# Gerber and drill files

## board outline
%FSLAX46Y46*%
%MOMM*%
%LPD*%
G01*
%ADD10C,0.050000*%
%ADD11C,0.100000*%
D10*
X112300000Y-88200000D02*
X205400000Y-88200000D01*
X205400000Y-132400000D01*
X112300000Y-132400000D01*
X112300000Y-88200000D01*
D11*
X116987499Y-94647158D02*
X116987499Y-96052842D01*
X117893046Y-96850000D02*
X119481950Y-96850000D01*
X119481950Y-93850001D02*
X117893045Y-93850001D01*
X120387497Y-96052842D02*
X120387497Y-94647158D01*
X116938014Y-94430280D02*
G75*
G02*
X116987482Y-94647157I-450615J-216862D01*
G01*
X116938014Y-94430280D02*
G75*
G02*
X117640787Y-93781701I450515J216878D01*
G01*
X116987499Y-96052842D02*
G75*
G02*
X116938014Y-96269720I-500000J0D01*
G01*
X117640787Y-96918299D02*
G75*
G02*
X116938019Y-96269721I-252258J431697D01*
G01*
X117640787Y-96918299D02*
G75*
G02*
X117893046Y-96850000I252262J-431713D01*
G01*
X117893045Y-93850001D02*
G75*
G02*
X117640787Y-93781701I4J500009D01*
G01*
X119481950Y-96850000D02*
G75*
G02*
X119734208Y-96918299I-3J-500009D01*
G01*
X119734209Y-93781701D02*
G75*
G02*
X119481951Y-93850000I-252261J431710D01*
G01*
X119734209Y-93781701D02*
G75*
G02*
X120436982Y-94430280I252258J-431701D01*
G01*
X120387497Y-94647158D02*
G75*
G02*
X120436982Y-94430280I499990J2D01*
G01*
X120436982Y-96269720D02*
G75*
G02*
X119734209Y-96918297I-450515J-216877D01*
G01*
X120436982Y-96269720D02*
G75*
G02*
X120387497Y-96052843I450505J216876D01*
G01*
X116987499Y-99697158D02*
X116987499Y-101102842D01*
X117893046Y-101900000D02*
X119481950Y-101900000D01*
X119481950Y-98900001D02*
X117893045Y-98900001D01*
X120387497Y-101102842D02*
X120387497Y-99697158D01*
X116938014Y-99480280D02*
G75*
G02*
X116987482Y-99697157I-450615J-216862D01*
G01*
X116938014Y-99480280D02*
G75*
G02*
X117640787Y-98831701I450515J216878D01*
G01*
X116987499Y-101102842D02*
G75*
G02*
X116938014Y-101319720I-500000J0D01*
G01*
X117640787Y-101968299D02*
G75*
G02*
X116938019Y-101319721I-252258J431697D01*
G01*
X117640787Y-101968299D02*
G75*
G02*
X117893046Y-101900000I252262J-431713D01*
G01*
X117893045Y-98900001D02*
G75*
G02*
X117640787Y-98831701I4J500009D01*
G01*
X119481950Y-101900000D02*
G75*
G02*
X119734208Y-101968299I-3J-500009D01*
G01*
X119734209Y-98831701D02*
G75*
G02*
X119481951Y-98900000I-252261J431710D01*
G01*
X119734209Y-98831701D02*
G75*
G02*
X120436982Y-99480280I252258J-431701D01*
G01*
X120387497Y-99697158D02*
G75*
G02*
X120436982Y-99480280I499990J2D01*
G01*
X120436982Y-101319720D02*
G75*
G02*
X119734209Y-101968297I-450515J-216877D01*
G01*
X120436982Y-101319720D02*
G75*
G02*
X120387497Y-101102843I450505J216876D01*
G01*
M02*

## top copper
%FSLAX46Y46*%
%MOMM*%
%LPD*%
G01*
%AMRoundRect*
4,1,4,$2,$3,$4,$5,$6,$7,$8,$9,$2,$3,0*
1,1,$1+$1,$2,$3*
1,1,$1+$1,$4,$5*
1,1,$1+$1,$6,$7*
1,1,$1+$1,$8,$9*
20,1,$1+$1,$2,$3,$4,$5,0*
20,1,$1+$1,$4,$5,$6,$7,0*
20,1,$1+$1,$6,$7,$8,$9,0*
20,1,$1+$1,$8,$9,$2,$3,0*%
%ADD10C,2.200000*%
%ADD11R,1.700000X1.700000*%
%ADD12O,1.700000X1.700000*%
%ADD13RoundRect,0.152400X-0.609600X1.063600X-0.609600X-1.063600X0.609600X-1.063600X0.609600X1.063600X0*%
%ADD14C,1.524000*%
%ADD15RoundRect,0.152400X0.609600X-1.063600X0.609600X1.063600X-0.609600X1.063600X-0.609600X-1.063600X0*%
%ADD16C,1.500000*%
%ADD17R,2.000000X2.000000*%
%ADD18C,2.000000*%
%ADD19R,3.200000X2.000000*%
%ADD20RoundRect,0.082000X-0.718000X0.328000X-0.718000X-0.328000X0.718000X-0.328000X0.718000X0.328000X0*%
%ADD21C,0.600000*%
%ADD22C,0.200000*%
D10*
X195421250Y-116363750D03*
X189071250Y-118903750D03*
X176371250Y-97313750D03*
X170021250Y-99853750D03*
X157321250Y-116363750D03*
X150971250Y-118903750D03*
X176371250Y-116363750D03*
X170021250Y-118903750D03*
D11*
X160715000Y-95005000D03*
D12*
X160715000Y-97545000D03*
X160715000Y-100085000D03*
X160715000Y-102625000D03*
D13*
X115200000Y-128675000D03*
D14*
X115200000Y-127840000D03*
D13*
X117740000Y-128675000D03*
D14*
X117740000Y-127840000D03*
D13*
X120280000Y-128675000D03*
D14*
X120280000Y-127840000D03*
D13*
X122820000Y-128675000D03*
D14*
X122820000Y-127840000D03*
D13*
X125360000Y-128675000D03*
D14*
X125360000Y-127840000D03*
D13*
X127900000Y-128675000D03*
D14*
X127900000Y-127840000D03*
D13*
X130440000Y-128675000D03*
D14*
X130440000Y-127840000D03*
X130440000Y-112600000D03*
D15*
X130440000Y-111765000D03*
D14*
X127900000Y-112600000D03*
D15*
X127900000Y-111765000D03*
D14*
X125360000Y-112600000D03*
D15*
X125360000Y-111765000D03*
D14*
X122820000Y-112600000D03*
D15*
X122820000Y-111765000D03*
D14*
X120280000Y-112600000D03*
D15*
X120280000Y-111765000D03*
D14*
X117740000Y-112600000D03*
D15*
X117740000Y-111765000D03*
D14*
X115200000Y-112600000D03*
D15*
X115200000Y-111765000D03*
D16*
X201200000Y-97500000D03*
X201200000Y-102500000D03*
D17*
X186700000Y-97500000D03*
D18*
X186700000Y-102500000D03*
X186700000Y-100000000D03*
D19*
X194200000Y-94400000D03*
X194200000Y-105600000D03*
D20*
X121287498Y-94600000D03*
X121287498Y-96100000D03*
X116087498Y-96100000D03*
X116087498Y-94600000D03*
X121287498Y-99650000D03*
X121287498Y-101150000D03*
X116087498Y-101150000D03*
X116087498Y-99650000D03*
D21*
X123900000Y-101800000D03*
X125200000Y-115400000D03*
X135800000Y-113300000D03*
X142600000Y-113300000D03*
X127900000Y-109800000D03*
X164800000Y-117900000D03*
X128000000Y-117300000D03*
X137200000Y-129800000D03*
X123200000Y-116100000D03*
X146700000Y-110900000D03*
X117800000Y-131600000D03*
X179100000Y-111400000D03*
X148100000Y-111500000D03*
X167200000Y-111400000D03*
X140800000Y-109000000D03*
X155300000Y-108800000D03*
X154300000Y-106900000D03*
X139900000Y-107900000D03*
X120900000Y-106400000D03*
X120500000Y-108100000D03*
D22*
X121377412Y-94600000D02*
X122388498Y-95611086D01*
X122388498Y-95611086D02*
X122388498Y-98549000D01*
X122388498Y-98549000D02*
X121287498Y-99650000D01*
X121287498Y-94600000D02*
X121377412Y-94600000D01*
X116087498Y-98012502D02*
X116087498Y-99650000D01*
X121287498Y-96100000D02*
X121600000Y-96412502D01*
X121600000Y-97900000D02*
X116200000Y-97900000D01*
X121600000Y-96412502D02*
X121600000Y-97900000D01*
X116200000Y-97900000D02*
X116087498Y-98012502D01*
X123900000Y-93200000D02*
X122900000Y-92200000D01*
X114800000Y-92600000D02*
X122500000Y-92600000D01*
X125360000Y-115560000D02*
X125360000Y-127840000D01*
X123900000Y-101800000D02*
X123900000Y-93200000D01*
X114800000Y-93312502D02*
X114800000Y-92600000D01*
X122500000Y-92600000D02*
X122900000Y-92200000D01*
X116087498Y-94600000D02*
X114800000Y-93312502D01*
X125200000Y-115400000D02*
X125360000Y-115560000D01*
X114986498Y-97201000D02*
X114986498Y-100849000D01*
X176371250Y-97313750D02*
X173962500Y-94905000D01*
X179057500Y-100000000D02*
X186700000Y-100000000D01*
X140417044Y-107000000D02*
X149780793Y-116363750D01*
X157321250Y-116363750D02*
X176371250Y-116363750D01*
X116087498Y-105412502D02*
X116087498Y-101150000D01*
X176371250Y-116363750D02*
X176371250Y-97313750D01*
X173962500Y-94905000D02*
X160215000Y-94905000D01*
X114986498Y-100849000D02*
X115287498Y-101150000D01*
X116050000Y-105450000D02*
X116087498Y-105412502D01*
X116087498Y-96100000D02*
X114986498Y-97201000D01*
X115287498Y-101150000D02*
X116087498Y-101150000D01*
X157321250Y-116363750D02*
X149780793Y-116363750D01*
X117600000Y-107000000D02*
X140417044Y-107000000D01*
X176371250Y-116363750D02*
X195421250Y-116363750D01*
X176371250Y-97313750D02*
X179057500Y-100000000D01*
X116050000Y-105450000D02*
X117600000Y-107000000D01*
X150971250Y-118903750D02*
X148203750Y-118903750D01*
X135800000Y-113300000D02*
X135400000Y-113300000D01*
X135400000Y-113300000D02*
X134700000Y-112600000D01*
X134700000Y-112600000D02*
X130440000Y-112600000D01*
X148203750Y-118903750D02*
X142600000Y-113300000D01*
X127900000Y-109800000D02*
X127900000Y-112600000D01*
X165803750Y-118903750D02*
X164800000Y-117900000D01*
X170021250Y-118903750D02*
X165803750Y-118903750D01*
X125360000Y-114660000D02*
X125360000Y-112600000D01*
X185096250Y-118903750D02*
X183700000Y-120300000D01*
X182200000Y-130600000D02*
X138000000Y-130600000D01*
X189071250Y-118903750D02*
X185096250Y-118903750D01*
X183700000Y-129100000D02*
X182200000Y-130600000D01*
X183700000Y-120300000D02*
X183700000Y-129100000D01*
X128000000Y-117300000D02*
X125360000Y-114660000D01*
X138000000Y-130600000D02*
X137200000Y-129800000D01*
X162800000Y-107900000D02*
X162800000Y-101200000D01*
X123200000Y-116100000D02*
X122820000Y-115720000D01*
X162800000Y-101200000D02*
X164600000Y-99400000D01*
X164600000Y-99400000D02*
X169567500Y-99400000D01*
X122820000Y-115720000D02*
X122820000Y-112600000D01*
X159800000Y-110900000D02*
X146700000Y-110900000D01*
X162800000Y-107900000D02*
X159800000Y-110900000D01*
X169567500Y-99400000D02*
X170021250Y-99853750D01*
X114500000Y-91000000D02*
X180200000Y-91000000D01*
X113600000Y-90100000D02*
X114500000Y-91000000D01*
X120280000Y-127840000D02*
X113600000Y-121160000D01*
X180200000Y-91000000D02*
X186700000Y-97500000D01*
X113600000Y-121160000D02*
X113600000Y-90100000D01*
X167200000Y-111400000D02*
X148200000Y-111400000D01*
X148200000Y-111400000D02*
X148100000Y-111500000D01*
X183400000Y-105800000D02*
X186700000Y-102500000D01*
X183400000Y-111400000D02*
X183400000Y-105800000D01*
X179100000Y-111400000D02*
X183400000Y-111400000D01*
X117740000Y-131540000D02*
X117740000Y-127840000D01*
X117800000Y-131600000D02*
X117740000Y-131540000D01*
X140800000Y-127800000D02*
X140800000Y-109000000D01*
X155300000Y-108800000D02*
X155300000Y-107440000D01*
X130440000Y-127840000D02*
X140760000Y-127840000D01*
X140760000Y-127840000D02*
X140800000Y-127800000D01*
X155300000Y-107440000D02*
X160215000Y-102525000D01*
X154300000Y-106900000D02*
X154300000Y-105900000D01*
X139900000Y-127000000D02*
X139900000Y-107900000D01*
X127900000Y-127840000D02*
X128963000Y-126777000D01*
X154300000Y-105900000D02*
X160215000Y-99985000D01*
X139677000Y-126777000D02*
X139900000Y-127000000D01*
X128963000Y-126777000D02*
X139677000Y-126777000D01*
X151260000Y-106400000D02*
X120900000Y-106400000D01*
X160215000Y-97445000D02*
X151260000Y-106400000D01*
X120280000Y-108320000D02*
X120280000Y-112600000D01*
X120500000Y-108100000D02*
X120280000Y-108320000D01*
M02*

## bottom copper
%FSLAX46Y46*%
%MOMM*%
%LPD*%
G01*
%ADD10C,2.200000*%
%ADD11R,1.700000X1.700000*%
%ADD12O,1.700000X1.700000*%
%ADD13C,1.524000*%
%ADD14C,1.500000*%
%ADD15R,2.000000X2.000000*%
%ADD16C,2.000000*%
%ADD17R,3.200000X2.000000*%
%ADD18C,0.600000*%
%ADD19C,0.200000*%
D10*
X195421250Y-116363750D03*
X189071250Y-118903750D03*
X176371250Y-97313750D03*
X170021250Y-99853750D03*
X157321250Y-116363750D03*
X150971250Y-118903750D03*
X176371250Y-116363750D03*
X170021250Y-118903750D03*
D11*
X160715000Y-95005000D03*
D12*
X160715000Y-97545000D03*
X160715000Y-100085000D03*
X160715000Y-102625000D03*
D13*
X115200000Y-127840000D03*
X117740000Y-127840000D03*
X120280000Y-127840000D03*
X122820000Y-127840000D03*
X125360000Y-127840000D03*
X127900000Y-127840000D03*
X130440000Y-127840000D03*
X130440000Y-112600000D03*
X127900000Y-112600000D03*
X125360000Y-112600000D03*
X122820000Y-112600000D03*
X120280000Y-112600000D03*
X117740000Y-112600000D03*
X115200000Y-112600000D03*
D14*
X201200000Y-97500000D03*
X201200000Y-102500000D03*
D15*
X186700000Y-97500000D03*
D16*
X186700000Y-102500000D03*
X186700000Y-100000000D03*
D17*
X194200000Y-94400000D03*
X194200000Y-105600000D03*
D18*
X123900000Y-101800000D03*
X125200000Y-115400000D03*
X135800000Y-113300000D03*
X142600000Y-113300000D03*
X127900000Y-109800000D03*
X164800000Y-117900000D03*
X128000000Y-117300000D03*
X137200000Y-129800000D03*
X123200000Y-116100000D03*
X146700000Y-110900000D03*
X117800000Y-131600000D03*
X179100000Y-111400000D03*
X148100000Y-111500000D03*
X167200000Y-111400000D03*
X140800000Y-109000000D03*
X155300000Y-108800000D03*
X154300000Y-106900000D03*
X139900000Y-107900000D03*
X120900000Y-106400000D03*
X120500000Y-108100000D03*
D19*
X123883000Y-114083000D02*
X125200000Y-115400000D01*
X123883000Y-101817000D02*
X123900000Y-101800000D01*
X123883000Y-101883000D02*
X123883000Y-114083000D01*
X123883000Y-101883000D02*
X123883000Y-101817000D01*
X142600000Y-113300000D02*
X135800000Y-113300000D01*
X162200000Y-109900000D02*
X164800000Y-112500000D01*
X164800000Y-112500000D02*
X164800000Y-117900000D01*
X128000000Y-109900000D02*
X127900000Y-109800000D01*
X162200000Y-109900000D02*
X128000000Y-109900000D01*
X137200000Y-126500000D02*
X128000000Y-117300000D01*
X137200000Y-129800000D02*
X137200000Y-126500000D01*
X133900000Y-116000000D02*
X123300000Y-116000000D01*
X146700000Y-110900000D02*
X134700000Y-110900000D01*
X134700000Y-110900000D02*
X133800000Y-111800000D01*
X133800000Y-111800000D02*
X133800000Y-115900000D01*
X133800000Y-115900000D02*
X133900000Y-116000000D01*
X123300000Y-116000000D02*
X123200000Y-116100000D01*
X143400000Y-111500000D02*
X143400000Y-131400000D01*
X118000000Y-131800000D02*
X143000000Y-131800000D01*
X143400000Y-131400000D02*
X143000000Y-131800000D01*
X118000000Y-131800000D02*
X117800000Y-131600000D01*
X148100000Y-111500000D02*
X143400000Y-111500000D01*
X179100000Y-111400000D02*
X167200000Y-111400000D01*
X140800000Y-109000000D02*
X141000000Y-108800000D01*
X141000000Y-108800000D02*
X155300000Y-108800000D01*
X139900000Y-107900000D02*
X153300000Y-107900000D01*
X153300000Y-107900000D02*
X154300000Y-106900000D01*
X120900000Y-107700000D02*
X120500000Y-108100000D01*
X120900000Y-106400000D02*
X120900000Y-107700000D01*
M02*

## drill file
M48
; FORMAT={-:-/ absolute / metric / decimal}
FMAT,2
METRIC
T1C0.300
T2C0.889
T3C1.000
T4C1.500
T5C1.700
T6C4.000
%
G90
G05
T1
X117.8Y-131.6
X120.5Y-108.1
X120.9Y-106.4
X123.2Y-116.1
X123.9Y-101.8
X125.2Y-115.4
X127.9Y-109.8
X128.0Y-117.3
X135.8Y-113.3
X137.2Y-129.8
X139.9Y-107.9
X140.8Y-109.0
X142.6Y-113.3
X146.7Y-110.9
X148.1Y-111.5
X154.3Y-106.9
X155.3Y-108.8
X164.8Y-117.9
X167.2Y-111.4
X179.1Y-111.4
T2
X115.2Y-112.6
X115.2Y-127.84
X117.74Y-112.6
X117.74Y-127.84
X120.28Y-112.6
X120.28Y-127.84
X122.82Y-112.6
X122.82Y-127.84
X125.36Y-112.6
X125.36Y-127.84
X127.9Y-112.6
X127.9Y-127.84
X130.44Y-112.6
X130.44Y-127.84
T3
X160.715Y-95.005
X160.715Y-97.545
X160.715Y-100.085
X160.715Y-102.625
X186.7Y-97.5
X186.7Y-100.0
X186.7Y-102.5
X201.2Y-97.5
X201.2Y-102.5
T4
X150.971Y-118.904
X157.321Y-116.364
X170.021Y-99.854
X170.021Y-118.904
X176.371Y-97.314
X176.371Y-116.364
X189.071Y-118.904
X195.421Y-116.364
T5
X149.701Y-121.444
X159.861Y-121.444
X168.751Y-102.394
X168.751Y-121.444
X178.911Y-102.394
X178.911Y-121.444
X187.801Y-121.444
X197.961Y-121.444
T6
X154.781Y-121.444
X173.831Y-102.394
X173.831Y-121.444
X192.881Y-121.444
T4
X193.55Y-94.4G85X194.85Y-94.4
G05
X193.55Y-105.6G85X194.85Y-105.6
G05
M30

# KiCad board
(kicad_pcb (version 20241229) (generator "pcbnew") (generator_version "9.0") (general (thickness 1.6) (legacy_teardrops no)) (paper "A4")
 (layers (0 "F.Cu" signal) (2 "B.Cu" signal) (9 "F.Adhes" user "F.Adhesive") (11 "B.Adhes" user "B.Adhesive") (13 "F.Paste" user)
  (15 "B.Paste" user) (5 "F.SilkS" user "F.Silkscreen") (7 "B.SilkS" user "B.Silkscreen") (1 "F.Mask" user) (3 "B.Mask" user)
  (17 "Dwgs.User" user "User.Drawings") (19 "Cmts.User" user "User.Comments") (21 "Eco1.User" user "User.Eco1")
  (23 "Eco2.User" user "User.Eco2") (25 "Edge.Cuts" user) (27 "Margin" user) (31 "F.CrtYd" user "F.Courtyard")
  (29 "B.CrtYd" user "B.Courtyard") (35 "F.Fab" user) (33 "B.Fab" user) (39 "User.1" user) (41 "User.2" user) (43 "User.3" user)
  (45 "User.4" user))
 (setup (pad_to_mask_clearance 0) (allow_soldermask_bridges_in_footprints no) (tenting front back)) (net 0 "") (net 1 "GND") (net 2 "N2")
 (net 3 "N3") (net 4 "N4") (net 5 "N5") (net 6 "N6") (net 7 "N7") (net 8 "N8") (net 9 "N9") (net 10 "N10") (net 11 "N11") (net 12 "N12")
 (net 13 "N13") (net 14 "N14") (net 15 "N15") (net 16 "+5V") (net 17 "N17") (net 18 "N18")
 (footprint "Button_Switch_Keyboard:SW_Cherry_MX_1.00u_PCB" (layer "F.Cu") (at 195.42125 116.36375)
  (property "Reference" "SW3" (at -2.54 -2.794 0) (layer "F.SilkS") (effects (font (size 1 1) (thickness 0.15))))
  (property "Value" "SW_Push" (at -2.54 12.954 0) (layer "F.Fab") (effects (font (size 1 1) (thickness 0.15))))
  (pad "" np_thru_hole circle (at -7.62 5.08) (size 1.7 1.7) (drill 1.7) (layers "*.Cu" "*.Mask"))
  (pad "" np_thru_hole circle (at -2.54 5.08) (size 4 4) (drill 4) (layers "*.Cu" "*.Mask"))
  (pad "" np_thru_hole circle (at 2.54 5.08) (size 1.7 1.7) (drill 1.7) (layers "*.Cu" "*.Mask"))
  (pad "1" thru_hole circle (at 0 0) (size 2.2 2.2) (drill 1.5) (layers "*.Cu" "*.Mask") (remove_unused_layers no) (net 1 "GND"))
  (pad "2" thru_hole circle (at -6.35 2.54) (size 2.2 2.2) (drill 1.5) (layers "*.Cu" "*.Mask") (remove_unused_layers no) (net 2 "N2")))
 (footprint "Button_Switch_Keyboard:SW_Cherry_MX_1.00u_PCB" (layer "F.Cu") (at 176.37125 97.31375)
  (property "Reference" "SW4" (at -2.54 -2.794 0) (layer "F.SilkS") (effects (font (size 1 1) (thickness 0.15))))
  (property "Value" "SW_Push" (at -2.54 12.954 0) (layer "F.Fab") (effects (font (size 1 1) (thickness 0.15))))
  (pad "" np_thru_hole circle (at -7.62 5.08) (size 1.7 1.7) (drill 1.7) (layers "*.Cu" "*.Mask"))
  (pad "" np_thru_hole circle (at -2.54 5.08) (size 4 4) (drill 4) (layers "*.Cu" "*.Mask"))
  (pad "" np_thru_hole circle (at 2.54 5.08) (size 1.7 1.7) (drill 1.7) (layers "*.Cu" "*.Mask"))
  (pad "1" thru_hole circle (at 0 0) (size 2.2 2.2) (drill 1.5) (layers "*.Cu" "*.Mask") (remove_unused_layers no) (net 1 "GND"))
  (pad "2" thru_hole circle (at -6.35 2.54) (size 2.2 2.2) (drill 1.5) (layers "*.Cu" "*.Mask") (remove_unused_layers no) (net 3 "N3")))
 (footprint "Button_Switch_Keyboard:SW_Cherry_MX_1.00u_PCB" (layer "F.Cu") (at 157.32125 116.36375)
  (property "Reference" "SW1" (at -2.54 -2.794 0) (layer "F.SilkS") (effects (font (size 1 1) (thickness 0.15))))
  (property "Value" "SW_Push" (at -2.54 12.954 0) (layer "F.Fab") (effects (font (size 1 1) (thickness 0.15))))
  (pad "" np_thru_hole circle (at -7.62 5.08) (size 1.7 1.7) (drill 1.7) (layers "*.Cu" "*.Mask"))
  (pad "" np_thru_hole circle (at -2.54 5.08) (size 4 4) (drill 4) (layers "*.Cu" "*.Mask"))
  (pad "" np_thru_hole circle (at 2.54 5.08) (size 1.7 1.7) (drill 1.7) (layers "*.Cu" "*.Mask"))
  (pad "1" thru_hole circle (at 0 0) (size 2.2 2.2) (drill 1.5) (layers "*.Cu" "*.Mask") (remove_unused_layers no) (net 1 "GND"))
  (pad "2" thru_hole circle (at -6.35 2.54) (size 2.2 2.2) (drill 1.5) (layers "*.Cu" "*.Mask") (remove_unused_layers no) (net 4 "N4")))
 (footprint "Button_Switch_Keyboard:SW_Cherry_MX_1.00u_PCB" (layer "F.Cu") (at 176.37125 116.36375)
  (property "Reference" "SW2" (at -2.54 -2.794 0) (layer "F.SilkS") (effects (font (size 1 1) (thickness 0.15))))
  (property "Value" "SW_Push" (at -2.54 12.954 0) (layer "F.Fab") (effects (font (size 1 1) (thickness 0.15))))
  (pad "" np_thru_hole circle (at -7.62 5.08) (size 1.7 1.7) (drill 1.7) (layers "*.Cu" "*.Mask"))
  (pad "" np_thru_hole circle (at -2.54 5.08) (size 4 4) (drill 4) (layers "*.Cu" "*.Mask"))
  (pad "" np_thru_hole circle (at 2.54 5.08) (size 1.7 1.7) (drill 1.7) (layers "*.Cu" "*.Mask"))
  (pad "1" thru_hole circle (at 0 0) (size 2.2 2.2) (drill 1.5) (layers "*.Cu" "*.Mask") (remove_unused_layers no) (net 1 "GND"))
  (pad "2" thru_hole circle (at -6.35 2.54) (size 2.2 2.2) (drill 1.5) (layers "*.Cu" "*.Mask") (remove_unused_layers no) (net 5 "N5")))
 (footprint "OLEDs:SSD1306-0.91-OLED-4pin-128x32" (layer "F.Cu") (at 124.215 92.815)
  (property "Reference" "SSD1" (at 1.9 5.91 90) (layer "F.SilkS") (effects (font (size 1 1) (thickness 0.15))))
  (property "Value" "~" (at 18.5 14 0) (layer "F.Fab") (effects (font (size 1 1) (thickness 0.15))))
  (pad "1" thru_hole rect (at 36.5 2.19) (size 1.7 1.7) (drill 1) (layers "*.Cu" "*.Mask") (remove_unused_layers no) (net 1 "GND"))
  (pad "2" thru_hole oval (at 36.5 4.73) (size 1.7 1.7) (drill 1) (layers "*.Cu" "*.Mask") (remove_unused_layers no) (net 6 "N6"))
  (pad "3" thru_hole oval (at 36.5 7.27) (size 1.7 1.7) (drill 1) (layers "*.Cu" "*.Mask") (remove_unused_layers no) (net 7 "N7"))
  (pad "4" thru_hole oval (at 36.5 9.81) (size 1.7 1.7) (drill 1) (layers "*.Cu" "*.Mask") (remove_unused_layers no) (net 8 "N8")))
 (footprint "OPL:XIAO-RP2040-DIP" (layer "F.Cu") (at 122.82 120.22 90)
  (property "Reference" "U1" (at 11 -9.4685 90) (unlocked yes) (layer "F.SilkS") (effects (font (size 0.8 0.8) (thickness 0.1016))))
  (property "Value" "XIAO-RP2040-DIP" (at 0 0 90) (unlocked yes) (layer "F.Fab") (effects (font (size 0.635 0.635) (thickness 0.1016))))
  (pad "1" smd roundrect (at -8.455 -7.62 270) (size 2.432 1.524) (layers "F.Cu" "F.Mask") (roundrect_rratio 0.1) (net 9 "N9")
   (thermal_bridge_angle 45))
  (pad "1" thru_hole circle (at -7.62 -7.62 270) (size 1.524 1.524) (drill 0.889) (layers "*.Cu" "*.Mask") (remove_unused_layers no)
   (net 9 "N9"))
  (pad "2" smd roundrect (at -8.455 -5.08 270) (size 2.432 1.524) (layers "F.Cu" "F.Mask") (roundrect_rratio 0.1) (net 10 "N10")
   (thermal_bridge_angle 45))
  (pad "2" thru_hole circle (at -7.62 -5.08 270) (size 1.524 1.524) (drill 0.889) (layers "*.Cu" "*.Mask") (remove_unused_layers no)
   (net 10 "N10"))
  (pad "3" smd roundrect (at -8.455 -2.54 270) (size 2.432 1.524) (layers "F.Cu" "F.Mask") (roundrect_rratio 0.1) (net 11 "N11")
   (thermal_bridge_angle 45))
  (pad "3" thru_hole circle (at -7.62 -2.54 270) (size 1.524 1.524) (drill 0.889) (layers "*.Cu" "*.Mask") (remove_unused_layers no)
   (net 11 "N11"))
  (pad "4" smd roundrect (at -8.455 0 270) (size 2.432 1.524) (layers "F.Cu" "F.Mask") (roundrect_rratio 0.1) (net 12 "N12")
   (thermal_bridge_angle 45))
  (pad "4" thru_hole circle (at -7.62 0 270) (size 1.524 1.524) (drill 0.889) (layers "*.Cu" "*.Mask") (remove_unused_layers no)
   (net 12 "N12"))
  (pad "5" smd roundrect (at -8.455 2.54 270) (size 2.432 1.524) (layers "F.Cu" "F.Mask") (roundrect_rratio 0.1) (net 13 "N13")
   (thermal_bridge_angle 45))
  (pad "5" thru_hole circle (at -7.62 2.54 270) (size 1.524 1.524) (drill 0.889) (layers "*.Cu" "*.Mask") (remove_unused_layers no)
   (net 13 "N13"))
  (pad "6" smd roundrect (at -8.455 5.08 270) (size 2.432 1.524) (layers "F.Cu" "F.Mask") (roundrect_rratio 0.1) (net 7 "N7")
   (thermal_bridge_angle 45))
  (pad "6" thru_hole circle (at -7.62 5.08 270) (size 1.524 1.524) (drill 0.889) (layers "*.Cu" "*.Mask") (remove_unused_layers no)
   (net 7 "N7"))
  (pad "7" smd roundrect (at -8.455 7.62 270) (size 2.432 1.524) (layers "F.Cu" "F.Mask") (roundrect_rratio 0.1) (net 8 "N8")
   (thermal_bridge_angle 45))
  (pad "7" thru_hole circle (at -7.62 7.62 270) (size 1.524 1.524) (drill 0.889) (layers "*.Cu" "*.Mask") (remove_unused_layers no)
   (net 8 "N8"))
  (pad "8" thru_hole circle (at 7.62 7.62 90) (size 1.524 1.524) (drill 0.889) (layers "*.Cu" "*.Mask") (remove_unused_layers no)
   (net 4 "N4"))
  (pad "8" smd roundrect (at 8.455 7.62 90) (size 2.432 1.524) (layers "F.Cu" "F.Mask") (roundrect_rratio 0.1) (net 4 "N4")
   (thermal_bridge_angle 45))
  (pad "9" thru_hole circle (at 7.62 5.08 90) (size 1.524 1.524) (drill 0.889) (layers "*.Cu" "*.Mask") (remove_unused_layers no)
   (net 5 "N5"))
  (pad "9" smd roundrect (at 8.455 5.08 90) (size 2.432 1.524) (layers "F.Cu" "F.Mask") (roundrect_rratio 0.1) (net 5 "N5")
   (thermal_bridge_angle 45))
  (pad "10" thru_hole circle (at 7.62 2.54 90) (size 1.524 1.524) (drill 0.889) (layers "*.Cu" "*.Mask") (remove_unused_layers no)
   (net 2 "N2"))
  (pad "10" smd roundrect (at 8.455 2.54 90) (size 2.432 1.524) (layers "F.Cu" "F.Mask") (roundrect_rratio 0.1) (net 2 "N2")
   (thermal_bridge_angle 45))
  (pad "11" thru_hole circle (at 7.62 0 90) (size 1.524 1.524) (drill 0.889) (layers "*.Cu" "*.Mask") (remove_unused_layers no) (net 3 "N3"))
  (pad "11" smd roundrect (at 8.455 0 90) (size 2.432 1.524) (layers "F.Cu" "F.Mask") (roundrect_rratio 0.1) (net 3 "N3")
   (thermal_bridge_angle 45))
  (pad "12" thru_hole circle (at 7.62 -2.54 90) (size 1.524 1.524) (drill 0.889) (layers "*.Cu" "*.Mask") (remove_unused_layers no)
   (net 6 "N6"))
  (pad "12" smd roundrect (at 8.455 -2.54 90) (size 2.432 1.524) (layers "F.Cu" "F.Mask") (roundrect_rratio 0.1) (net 6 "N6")
   (thermal_bridge_angle 45))
  (pad "13" thru_hole circle (at 7.62 -5.08 90) (size 1.524 1.524) (drill 0.889) (layers "*.Cu" "*.Mask") (remove_unused_layers no)
   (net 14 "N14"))
  (pad "13" smd roundrect (at 8.455 -5.08 90) (size 2.432 1.524) (layers "F.Cu" "F.Mask") (roundrect_rratio 0.1) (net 14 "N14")
   (thermal_bridge_angle 45))
  (pad "14" thru_hole circle (at 7.62 -7.62 90) (size 1.524 1.524) (drill 0.889) (layers "*.Cu" "*.Mask") (remove_unused_layers no)
   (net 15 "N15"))
  (pad "14" smd roundrect (at 8.455 -7.62 90) (size 2.432 1.524) (layers "F.Cu" "F.Mask") (roundrect_rratio 0.1) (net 15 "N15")
   (thermal_bridge_angle 45)))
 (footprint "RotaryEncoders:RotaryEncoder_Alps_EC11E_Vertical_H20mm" (layer "F.Cu") (at 186.7 97.5)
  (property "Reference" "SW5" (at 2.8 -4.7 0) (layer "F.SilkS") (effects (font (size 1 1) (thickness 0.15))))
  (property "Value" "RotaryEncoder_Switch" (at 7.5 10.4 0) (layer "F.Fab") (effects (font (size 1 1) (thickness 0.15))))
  (pad "" thru_hole circle (at 14.5 0) (size 1.5 1.5) (drill 1) (layers "*.Cu" "*.Mask") (remove_unused_layers no))
  (pad "" thru_hole circle (at 14.5 5) (size 1.5 1.5) (drill 1) (layers "*.Cu" "*.Mask") (remove_unused_layers no))
  (pad "A" thru_hole rect (at 0 0) (size 2 2) (drill 1) (layers "*.Cu" "*.Mask") (remove_unused_layers no) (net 11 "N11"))
  (pad "B" thru_hole circle (at 0 5) (size 2 2) (drill 1) (layers "*.Cu" "*.Mask") (remove_unused_layers no) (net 10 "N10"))
  (pad "C" thru_hole circle (at 0 2.5) (size 2 2) (drill 1) (layers "*.Cu" "*.Mask") (remove_unused_layers no) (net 1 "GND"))
  (pad "MP" thru_hole rect (at 7.5 -3.1) (size 3.2 2) (drill oval 2.8 1.5) (layers "*.Cu" "*.Mask") (remove_unused_layers no))
  (pad "MP" thru_hole rect (at 7.5 8.1) (size 3.2 2) (drill oval 2.8 1.5) (layers "*.Cu" "*.Mask") (remove_unused_layers no)))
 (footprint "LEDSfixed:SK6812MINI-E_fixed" (layer "B.Cu") (at 118.687499 95.452842 180)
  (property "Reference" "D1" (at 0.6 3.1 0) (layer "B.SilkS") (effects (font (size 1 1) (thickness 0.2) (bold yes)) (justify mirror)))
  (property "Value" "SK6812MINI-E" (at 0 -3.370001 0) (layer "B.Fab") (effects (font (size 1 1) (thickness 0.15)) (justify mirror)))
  (fp_line (start 1.7 0.805684) (end 1.7 -0.6) (stroke (width 0.1) (type solid)) (layer "Edge.Cuts"))
  (fp_line (start 0.794453 -1.397158) (end -0.794451 -1.397158) (stroke (width 0.1) (type solid)) (layer "Edge.Cuts"))
  (fp_line (start -0.794451 1.602841) (end 0.794454 1.602841) (stroke (width 0.1) (type solid)) (layer "Edge.Cuts"))
  (fp_line (start -1.699998 -0.6) (end -1.699998 0.805684) (stroke (width 0.1) (type solid)) (layer "Edge.Cuts"))
  (fp_arc (start 1.749485 1.022562) (mid 1.712532 0.91691) (end 1.7 0.805685) (stroke (width 0.1) (type solid)) (layer "Edge.Cuts"))
  (fp_arc (start 1.749485 1.022562) (mid 1.638072 1.606877) (end 1.046712 1.67114) (stroke (width 0.1) (type solid)) (layer "Edge.Cuts"))
  (fp_arc (start 1.7 -0.6) (mid 1.712528 -0.711226) (end 1.749485 -0.816878) (stroke (width 0.1) (type solid)) (layer "Edge.Cuts"))
  (fp_arc (start 1.046712 -1.465457) (mid 1.638073 -1.401193) (end 1.749485 -0.816877) (stroke (width 0.1) (type solid)) (layer "Edge.Cuts"))
  (fp_arc (start 1.046712 -1.465457) (mid 0.925124 -1.414535) (end 0.794453 -1.397158) (stroke (width 0.1) (type solid)) (layer "Edge.Cuts"))
  (fp_arc (start 0.794454 1.602841) (mid 0.925124 1.620218) (end 1.046712 1.67114) (stroke (width 0.1) (type solid)) (layer "Edge.Cuts"))
  (fp_arc (start -0.794451 -1.397158) (mid -0.925121 -1.414535) (end -1.046709 -1.465457) (stroke (width 0.1) (type solid))
   (layer "Edge.Cuts"))
  (fp_arc (start -1.04671 1.671141) (mid -0.925122 1.620219) (end -0.794452 1.602842) (stroke (width 0.1) (type solid)) (layer "Edge.Cuts"))
  (fp_arc (start -1.04671 1.671141) (mid -1.63807 1.606877) (end -1.749483 1.022562) (stroke (width 0.1) (type solid)) (layer "Edge.Cuts"))
  (fp_arc (start -1.699998 0.805684) (mid -1.712526 0.91691) (end -1.749483 1.022562) (stroke (width 0.1) (type solid)) (layer "Edge.Cuts"))
  (fp_arc (start -1.749483 -0.816878) (mid -1.638069 -1.401192) (end -1.04671 -1.465455) (stroke (width 0.1) (type solid))
   (layer "Edge.Cuts"))
  (fp_arc (start -1.749483 -0.816878) (mid -1.712526 -0.711226) (end -1.699998 -0.600001) (stroke (width 0.1) (type solid))
   (layer "Edge.Cuts"))
  (pad "1" smd roundrect (at -2.599999 0.852842 270) (size 0.82 1.6) (layers "F.Cu" "F.Mask" "F.Paste") (roundrect_rratio 0.1)
   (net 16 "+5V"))
  (pad "2" smd roundrect (at -2.599999 -0.647158 270) (size 0.82 1.6) (layers "F.Cu" "F.Mask" "F.Paste") (roundrect_rratio 0.1)
   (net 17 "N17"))
  (pad "3" smd roundrect (at 2.600001 -0.647158 270) (size 0.82 1.6) (layers "F.Cu" "F.Mask" "F.Paste") (roundrect_rratio 0.1) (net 1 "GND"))
  (pad "4" smd roundrect (at 2.600001 0.852842 270) (size 0.82 1.6) (layers "F.Cu" "F.Mask" "F.Paste") (roundrect_rratio 0.1) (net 13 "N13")))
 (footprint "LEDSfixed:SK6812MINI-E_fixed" (layer "B.Cu") (at 118.687499 100.502842 180)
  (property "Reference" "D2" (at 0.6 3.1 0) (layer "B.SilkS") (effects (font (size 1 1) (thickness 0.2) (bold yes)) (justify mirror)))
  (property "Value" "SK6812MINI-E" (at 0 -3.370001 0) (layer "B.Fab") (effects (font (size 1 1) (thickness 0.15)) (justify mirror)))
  (fp_line (start 1.7 0.805684) (end 1.7 -0.6) (stroke (width 0.1) (type solid)) (layer "Edge.Cuts"))
  (fp_line (start 0.794453 -1.397158) (end -0.794451 -1.397158) (stroke (width 0.1) (type solid)) (layer "Edge.Cuts"))
  (fp_line (start -0.794451 1.602841) (end 0.794454 1.602841) (stroke (width 0.1) (type solid)) (layer "Edge.Cuts"))
  (fp_line (start -1.699998 -0.6) (end -1.699998 0.805684) (stroke (width 0.1) (type solid)) (layer "Edge.Cuts"))
  (fp_arc (start 1.749485 1.022562) (mid 1.712532 0.91691) (end 1.7 0.805685) (stroke (width 0.1) (type solid)) (layer "Edge.Cuts"))
  (fp_arc (start 1.749485 1.022562) (mid 1.638072 1.606877) (end 1.046712 1.67114) (stroke (width 0.1) (type solid)) (layer "Edge.Cuts"))
  (fp_arc (start 1.7 -0.6) (mid 1.712528 -0.711226) (end 1.749485 -0.816878) (stroke (width 0.1) (type solid)) (layer "Edge.Cuts"))
  (fp_arc (start 1.046712 -1.465457) (mid 1.638073 -1.401193) (end 1.749485 -0.816877) (stroke (width 0.1) (type solid)) (layer "Edge.Cuts"))
  (fp_arc (start 1.046712 -1.465457) (mid 0.925124 -1.414535) (end 0.794453 -1.397158) (stroke (width 0.1) (type solid)) (layer "Edge.Cuts"))
  (fp_arc (start 0.794454 1.602841) (mid 0.925124 1.620218) (end 1.046712 1.67114) (stroke (width 0.1) (type solid)) (layer "Edge.Cuts"))
  (fp_arc (start -0.794451 -1.397158) (mid -0.925121 -1.414535) (end -1.046709 -1.465457) (stroke (width 0.1) (type solid))
   (layer "Edge.Cuts"))
  (fp_arc (start -1.04671 1.671141) (mid -0.925122 1.620219) (end -0.794452 1.602842) (stroke (width 0.1) (type solid)) (layer "Edge.Cuts"))
  (fp_arc (start -1.04671 1.671141) (mid -1.63807 1.606877) (end -1.749483 1.022562) (stroke (width 0.1) (type solid)) (layer "Edge.Cuts"))
  (fp_arc (start -1.699998 0.805684) (mid -1.712526 0.91691) (end -1.749483 1.022562) (stroke (width 0.1) (type solid)) (layer "Edge.Cuts"))
  (fp_arc (start -1.749483 -0.816878) (mid -1.638069 -1.401192) (end -1.04671 -1.465455) (stroke (width 0.1) (type solid))
   (layer "Edge.Cuts"))
  (fp_arc (start -1.749483 -0.816878) (mid -1.712526 -0.711226) (end -1.699998 -0.600001) (stroke (width 0.1) (type solid))
   (layer "Edge.Cuts"))
  (pad "1" smd roundrect (at -2.599999 0.852842 270) (size 0.82 1.6) (layers "F.Cu" "F.Mask" "F.Paste") (roundrect_rratio 0.1)
   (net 16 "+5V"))
  (pad "2" smd roundrect (at -2.599999 -0.647158 270) (size 0.82 1.6) (layers "F.Cu" "F.Mask" "F.Paste") (roundrect_rratio 0.1)
   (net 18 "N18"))
  (pad "3" smd roundrect (at 2.600001 -0.647158 270) (size 0.82 1.6) (layers "F.Cu" "F.Mask" "F.Paste") (roundrect_rratio 0.1) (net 1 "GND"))
  (pad "4" smd roundrect (at 2.600001 0.852842 270) (size 0.82 1.6) (layers "F.Cu" "F.Mask" "F.Paste") (roundrect_rratio 0.1) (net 17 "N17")))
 (gr_rect (start 112.3 88.2) (end 205.4 132.4) (stroke (width 0.05) (type default)) (fill no) (layer "Edge.Cuts"))
 (segment (start 121.377412 94.6) (end 122.388498 95.611086) (width 0.2) (layer "F.Cu") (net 16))
 (segment (start 122.388498 95.611086) (end 122.388498 98.549) (width 0.2) (layer "F.Cu") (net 16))
 (segment (start 122.388498 98.549) (end 121.287498 99.65) (width 0.2) (layer "F.Cu") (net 16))
 (segment (start 121.287498 94.6) (end 121.377412 94.6) (width 0.2) (layer "F.Cu") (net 16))
 (segment (start 116.087498 98.012502) (end 116.087498 99.65) (width 0.2) (layer "F.Cu") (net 17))
 (segment (start 121.287498 96.1) (end 121.6 96.412502) (width 0.2) (layer "F.Cu") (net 17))
 (segment (start 121.6 97.9) (end 116.2 97.9) (width 0.2) (layer "F.Cu") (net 17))
 (segment (start 121.6 96.412502) (end 121.6 97.9) (width 0.2) (layer "F.Cu") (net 17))
 (segment (start 116.2 97.9) (end 116.087498 98.012502) (width 0.2) (layer "F.Cu") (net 17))
 (segment (start 123.9 93.2) (end 122.9 92.2) (width 0.2) (layer "F.Cu") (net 13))
 (segment (start 114.8 92.6) (end 122.5 92.6) (width 0.2) (layer "F.Cu") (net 13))
 (segment (start 125.36 115.56) (end 125.36 127.84) (width 0.2) (layer "F.Cu") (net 13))
 (segment (start 123.9 101.8) (end 123.9 93.2) (width 0.2) (layer "F.Cu") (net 13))
 (segment (start 114.8 93.312502) (end 114.8 92.6) (width 0.2) (layer "F.Cu") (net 13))
 (segment (start 122.5 92.6) (end 122.9 92.2) (width 0.2) (layer "F.Cu") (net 13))
 (segment (start 116.087498 94.6) (end 114.8 93.312502) (width 0.2) (layer "F.Cu") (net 13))
 (segment (start 125.2 115.4) (end 125.36 115.56) (width 0.2) (layer "F.Cu") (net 13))
 (via (at 123.9 101.8) (size 0.6) (drill 0.3) (layers "F.Cu" "B.Cu") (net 13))
 (via (at 125.2 115.4) (size 0.6) (drill 0.3) (layers "F.Cu" "B.Cu") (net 13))
 (segment (start 123.883 114.083) (end 125.2 115.4) (width 0.2) (layer "B.Cu") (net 13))
 (segment (start 123.883 101.817) (end 123.9 101.8) (width 0.2) (layer "B.Cu") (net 13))
 (segment (start 123.883 101.883) (end 123.883 114.083) (width 0.2) (layer "B.Cu") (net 13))
 (segment (start 123.883 101.883) (end 123.883 101.817) (width 0.2) (layer "B.Cu") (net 13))
 (segment (start 114.986498 97.201) (end 114.986498 100.849) (width 0.2) (layer "F.Cu") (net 1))
 (segment (start 176.37125 97.31375) (end 173.9625 94.905) (width 0.2) (layer "F.Cu") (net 1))
 (segment (start 179.0575 100) (end 186.7 100) (width 0.2) (layer "F.Cu") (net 1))
 (segment (start 140.417044 107) (end 149.780793 116.36375) (width 0.2) (layer "F.Cu") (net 1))
 (segment (start 157.32125 116.36375) (end 176.37125 116.36375) (width 0.2) (layer "F.Cu") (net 1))
 (segment (start 116.087498 105.412502) (end 116.087498 101.15) (width 0.2) (layer "F.Cu") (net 1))
 (segment (start 176.37125 116.36375) (end 176.37125 97.31375) (width 0.2) (layer "F.Cu") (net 1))
 (segment (start 173.9625 94.905) (end 160.215 94.905) (width 0.2) (layer "F.Cu") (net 1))
 (segment (start 114.986498 100.849) (end 115.287498 101.15) (width 0.2) (layer "F.Cu") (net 1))
 (segment (start 116.05 105.45) (end 116.087498 105.412502) (width 0.2) (layer "F.Cu") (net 1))
 (segment (start 116.087498 96.1) (end 114.986498 97.201) (width 0.2) (layer "F.Cu") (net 1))
 (segment (start 115.287498 101.15) (end 116.087498 101.15) (width 0.2) (layer "F.Cu") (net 1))
 (segment (start 157.32125 116.36375) (end 149.780793 116.36375) (width 0.2) (layer "F.Cu") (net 1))
 (segment (start 117.6 107) (end 140.417044 107) (width 0.2) (layer "F.Cu") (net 1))
 (segment (start 176.37125 116.36375) (end 195.42125 116.36375) (width 0.2) (layer "F.Cu") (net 1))
 (segment (start 176.37125 97.31375) (end 179.0575 100) (width 0.2) (layer "F.Cu") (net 1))
 (segment (start 116.05 105.45) (end 117.6 107) (width 0.2) (layer "F.Cu") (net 1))
 (segment (start 150.97125 118.90375) (end 148.20375 118.90375) (width 0.2) (layer "F.Cu") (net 4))
 (segment (start 135.8 113.3) (end 135.4 113.3) (width 0.2) (layer "F.Cu") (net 4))
 (segment (start 135.4 113.3) (end 134.7 112.6) (width 0.2) (layer "F.Cu") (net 4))
 (segment (start 134.7 112.6) (end 130.44 112.6) (width 0.2) (layer "F.Cu") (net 4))
 (segment (start 148.20375 118.90375) (end 142.6 113.3) (width 0.2) (layer "F.Cu") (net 4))
 (via (at 135.8 113.3) (size 0.6) (drill 0.3) (layers "F.Cu" "B.Cu") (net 4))
 (via (at 142.6 113.3) (size 0.6) (drill 0.3) (layers "F.Cu" "B.Cu") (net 4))
 (segment (start 142.6 113.3) (end 135.8 113.3) (width 0.2) (layer "B.Cu") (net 4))
 (segment (start 127.9 109.8) (end 127.9 112.6) (width 0.2) (layer "F.Cu") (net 5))
 (segment (start 165.80375 118.90375) (end 164.8 117.9) (width 0.2) (layer "F.Cu") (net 5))
 (segment (start 170.02125 118.90375) (end 165.80375 118.90375) (width 0.2) (layer "F.Cu") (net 5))
 (via (at 127.9 109.8) (size 0.6) (drill 0.3) (layers "F.Cu" "B.Cu") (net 5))
 (via (at 164.8 117.9) (size 0.6) (drill 0.3) (layers "F.Cu" "B.Cu") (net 5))
 (segment (start 162.2 109.9) (end 164.8 112.5) (width 0.2) (layer "B.Cu") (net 5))
 (segment (start 164.8 112.5) (end 164.8 117.9) (width 0.2) (layer "B.Cu") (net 5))
 (segment (start 128 109.9) (end 127.9 109.8) (width 0.2) (layer "B.Cu") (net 5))
 (segment (start 162.2 109.9) (end 128 109.9) (width 0.2) (layer "B.Cu") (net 5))
 (segment (start 125.36 114.66) (end 125.36 112.6) (width 0.2) (layer "F.Cu") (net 2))
 (segment (start 185.09625 118.90375) (end 183.7 120.3) (width 0.2) (layer "F.Cu") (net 2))
 (segment (start 182.2 130.6) (end 138 130.6) (width 0.2) (layer "F.Cu") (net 2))
 (segment (start 189.07125 118.90375) (end 185.09625 118.90375) (width 0.2) (layer "F.Cu") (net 2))
 (segment (start 183.7 129.1) (end 182.2 130.6) (width 0.2) (layer "F.Cu") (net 2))
 (segment (start 183.7 120.3) (end 183.7 129.1) (width 0.2) (layer "F.Cu") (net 2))
 (segment (start 128 117.3) (end 125.36 114.66) (width 0.2) (layer "F.Cu") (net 2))
 (segment (start 138 130.6) (end 137.2 129.8) (width 0.2) (layer "F.Cu") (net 2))
 (via (at 128 117.3) (size 0.6) (drill 0.3) (layers "F.Cu" "B.Cu") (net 2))
 (via (at 137.2 129.8) (size 0.6) (drill 0.3) (layers "F.Cu" "B.Cu") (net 2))
 (segment (start 137.2 126.5) (end 128 117.3) (width 0.2) (layer "B.Cu") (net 2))
 (segment (start 137.2 129.8) (end 137.2 126.5) (width 0.2) (layer "B.Cu") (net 2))
 (segment (start 162.8 107.9) (end 162.8 101.2) (width 0.2) (layer "F.Cu") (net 3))
 (segment (start 123.2 116.1) (end 122.82 115.72) (width 0.2) (layer "F.Cu") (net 3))
 (segment (start 162.8 101.2) (end 164.6 99.4) (width 0.2) (layer "F.Cu") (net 3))
 (segment (start 164.6 99.4) (end 169.5675 99.4) (width 0.2) (layer "F.Cu") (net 3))
 (segment (start 122.82 115.72) (end 122.82 112.6) (width 0.2) (layer "F.Cu") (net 3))
 (segment (start 159.8 110.9) (end 146.7 110.9) (width 0.2) (layer "F.Cu") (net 3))
 (segment (start 162.8 107.9) (end 159.8 110.9) (width 0.2) (layer "F.Cu") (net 3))
 (segment (start 169.5675 99.4) (end 170.02125 99.85375) (width 0.2) (layer "F.Cu") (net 3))
 (via (at 123.2 116.1) (size 0.6) (drill 0.3) (layers "F.Cu" "B.Cu") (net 3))
 (via (at 146.7 110.9) (size 0.6) (drill 0.3) (layers "F.Cu" "B.Cu") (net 3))
 (segment (start 133.9 116) (end 123.3 116) (width 0.2) (layer "B.Cu") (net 3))
 (segment (start 146.7 110.9) (end 134.7 110.9) (width 0.2) (layer "B.Cu") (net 3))
 (segment (start 134.7 110.9) (end 133.8 111.8) (width 0.2) (layer "B.Cu") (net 3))
 (segment (start 133.8 111.8) (end 133.8 115.9) (width 0.2) (layer "B.Cu") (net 3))
 (segment (start 133.8 115.9) (end 133.9 116) (width 0.2) (layer "B.Cu") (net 3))
 (segment (start 123.3 116) (end 123.2 116.1) (width 0.2) (layer "B.Cu") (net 3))
 (segment (start 114.5 91) (end 180.2 91) (width 0.2) (layer "F.Cu") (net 11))
 (segment (start 113.6 90.1) (end 114.5 91) (width 0.2) (layer "F.Cu") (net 11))
 (segment (start 120.28 127.84) (end 113.6 121.16) (width 0.2) (layer "F.Cu") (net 11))
 (segment (start 180.2 91) (end 186.7 97.5) (width 0.2) (layer "F.Cu") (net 11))
 (segment (start 113.6 121.16) (end 113.6 90.1) (width 0.2) (layer "F.Cu") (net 11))
 (segment (start 167.2 111.4) (end 148.2 111.4) (width 0.2) (layer "F.Cu") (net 10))
 (segment (start 148.2 111.4) (end 148.1 111.5) (width 0.2) (layer "F.Cu") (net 10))
 (segment (start 183.4 105.8) (end 186.7 102.5) (width 0.2) (layer "F.Cu") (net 10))
 (segment (start 183.4 111.4) (end 183.4 105.8) (width 0.2) (layer "F.Cu") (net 10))
 (segment (start 179.1 111.4) (end 183.4 111.4) (width 0.2) (layer "F.Cu") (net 10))
 (segment (start 117.74 131.54) (end 117.74 127.84) (width 0.2) (layer "F.Cu") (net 10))
 (segment (start 117.8 131.6) (end 117.74 131.54) (width 0.2) (layer "F.Cu") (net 10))
 (via (at 117.8 131.6) (size 0.6) (drill 0.3) (layers "F.Cu" "B.Cu") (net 10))
 (via (at 179.1 111.4) (size 0.6) (drill 0.3) (layers "F.Cu" "B.Cu") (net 10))
 (via (at 148.1 111.5) (size 0.6) (drill 0.3) (layers "F.Cu" "B.Cu") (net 10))
 (via (at 167.2 111.4) (size 0.6) (drill 0.3) (layers "F.Cu" "B.Cu") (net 10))
 (segment (start 143.4 111.5) (end 143.4 131.4) (width 0.2) (layer "B.Cu") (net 10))
 (segment (start 118 131.8) (end 143 131.8) (width 0.2) (layer "B.Cu") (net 10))
 (segment (start 143.4 131.4) (end 143 131.8) (width 0.2) (layer "B.Cu") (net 10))
 (segment (start 118 131.8) (end 117.8 131.6) (width 0.2) (layer "B.Cu") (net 10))
 (segment (start 148.1 111.5) (end 143.4 111.5) (width 0.2) (layer "B.Cu") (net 10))
 (segment (start 179.1 111.4) (end 167.2 111.4) (width 0.2) (layer "B.Cu") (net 10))
 (segment (start 140.8 127.8) (end 140.8 109) (width 0.2) (layer "F.Cu") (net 8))
 (segment (start 155.3 108.8) (end 155.3 107.44) (width 0.2) (layer "F.Cu") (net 8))
 (segment (start 130.44 127.84) (end 140.76 127.84) (width 0.2) (layer "F.Cu") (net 8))
 (segment (start 140.76 127.84) (end 140.8 127.8) (width 0.2) (layer "F.Cu") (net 8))
 (segment (start 155.3 107.44) (end 160.215 102.525) (width 0.2) (layer "F.Cu") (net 8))
 (via (at 140.8 109) (size 0.6) (drill 0.3) (layers "F.Cu" "B.Cu") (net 8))
 (via (at 155.3 108.8) (size 0.6) (drill 0.3) (layers "F.Cu" "B.Cu") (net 8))
 (segment (start 140.8 109) (end 141 108.8) (width 0.2) (layer "B.Cu") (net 8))
 (segment (start 141 108.8) (end 155.3 108.8) (width 0.2) (layer "B.Cu") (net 8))
 (segment (start 154.3 106.9) (end 154.3 105.9) (width 0.2) (layer "F.Cu") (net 7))
 (segment (start 139.9 127) (end 139.9 107.9) (width 0.2) (layer "F.Cu") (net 7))
 (segment (start 127.9 127.84) (end 128.963 126.777) (width 0.2) (layer "F.Cu") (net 7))
 (segment (start 154.3 105.9) (end 160.215 99.985) (width 0.2) (layer "F.Cu") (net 7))
 (segment (start 139.677 126.777) (end 139.9 127) (width 0.2) (layer "F.Cu") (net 7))
 (segment (start 128.963 126.777) (end 139.677 126.777) (width 0.2) (layer "F.Cu") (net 7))
 (via (at 154.3 106.9) (size 0.6) (drill 0.3) (layers "F.Cu" "B.Cu") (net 7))
 (via (at 139.9 107.9) (size 0.6) (drill 0.3) (layers "F.Cu" "B.Cu") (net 7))
 (segment (start 139.9 107.9) (end 153.3 107.9) (width 0.2) (layer "B.Cu") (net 7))
 (segment (start 153.3 107.9) (end 154.3 106.9) (width 0.2) (layer "B.Cu") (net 7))
 (segment (start 151.26 106.4) (end 120.9 106.4) (width 0.2) (layer "F.Cu") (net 6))
 (segment (start 160.215 97.445) (end 151.26 106.4) (width 0.2) (layer "F.Cu") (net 6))
 (segment (start 120.28 108.32) (end 120.28 112.6) (width 0.2) (layer "F.Cu") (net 6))
 (segment (start 120.5 108.1) (end 120.28 108.32) (width 0.2) (layer "F.Cu") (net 6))
 (via (at 120.9 106.4) (size 0.6) (drill 0.3) (layers "F.Cu" "B.Cu") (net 6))
 (via (at 120.5 108.1) (size 0.6) (drill 0.3) (layers "F.Cu" "B.Cu") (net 6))
 (segment (start 120.9 107.7) (end 120.5 108.1) (width 0.2) (layer "B.Cu") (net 6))
 (segment (start 120.9 106.4) (end 120.9 107.7) (width 0.2) (layer "B.Cu") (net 6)))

